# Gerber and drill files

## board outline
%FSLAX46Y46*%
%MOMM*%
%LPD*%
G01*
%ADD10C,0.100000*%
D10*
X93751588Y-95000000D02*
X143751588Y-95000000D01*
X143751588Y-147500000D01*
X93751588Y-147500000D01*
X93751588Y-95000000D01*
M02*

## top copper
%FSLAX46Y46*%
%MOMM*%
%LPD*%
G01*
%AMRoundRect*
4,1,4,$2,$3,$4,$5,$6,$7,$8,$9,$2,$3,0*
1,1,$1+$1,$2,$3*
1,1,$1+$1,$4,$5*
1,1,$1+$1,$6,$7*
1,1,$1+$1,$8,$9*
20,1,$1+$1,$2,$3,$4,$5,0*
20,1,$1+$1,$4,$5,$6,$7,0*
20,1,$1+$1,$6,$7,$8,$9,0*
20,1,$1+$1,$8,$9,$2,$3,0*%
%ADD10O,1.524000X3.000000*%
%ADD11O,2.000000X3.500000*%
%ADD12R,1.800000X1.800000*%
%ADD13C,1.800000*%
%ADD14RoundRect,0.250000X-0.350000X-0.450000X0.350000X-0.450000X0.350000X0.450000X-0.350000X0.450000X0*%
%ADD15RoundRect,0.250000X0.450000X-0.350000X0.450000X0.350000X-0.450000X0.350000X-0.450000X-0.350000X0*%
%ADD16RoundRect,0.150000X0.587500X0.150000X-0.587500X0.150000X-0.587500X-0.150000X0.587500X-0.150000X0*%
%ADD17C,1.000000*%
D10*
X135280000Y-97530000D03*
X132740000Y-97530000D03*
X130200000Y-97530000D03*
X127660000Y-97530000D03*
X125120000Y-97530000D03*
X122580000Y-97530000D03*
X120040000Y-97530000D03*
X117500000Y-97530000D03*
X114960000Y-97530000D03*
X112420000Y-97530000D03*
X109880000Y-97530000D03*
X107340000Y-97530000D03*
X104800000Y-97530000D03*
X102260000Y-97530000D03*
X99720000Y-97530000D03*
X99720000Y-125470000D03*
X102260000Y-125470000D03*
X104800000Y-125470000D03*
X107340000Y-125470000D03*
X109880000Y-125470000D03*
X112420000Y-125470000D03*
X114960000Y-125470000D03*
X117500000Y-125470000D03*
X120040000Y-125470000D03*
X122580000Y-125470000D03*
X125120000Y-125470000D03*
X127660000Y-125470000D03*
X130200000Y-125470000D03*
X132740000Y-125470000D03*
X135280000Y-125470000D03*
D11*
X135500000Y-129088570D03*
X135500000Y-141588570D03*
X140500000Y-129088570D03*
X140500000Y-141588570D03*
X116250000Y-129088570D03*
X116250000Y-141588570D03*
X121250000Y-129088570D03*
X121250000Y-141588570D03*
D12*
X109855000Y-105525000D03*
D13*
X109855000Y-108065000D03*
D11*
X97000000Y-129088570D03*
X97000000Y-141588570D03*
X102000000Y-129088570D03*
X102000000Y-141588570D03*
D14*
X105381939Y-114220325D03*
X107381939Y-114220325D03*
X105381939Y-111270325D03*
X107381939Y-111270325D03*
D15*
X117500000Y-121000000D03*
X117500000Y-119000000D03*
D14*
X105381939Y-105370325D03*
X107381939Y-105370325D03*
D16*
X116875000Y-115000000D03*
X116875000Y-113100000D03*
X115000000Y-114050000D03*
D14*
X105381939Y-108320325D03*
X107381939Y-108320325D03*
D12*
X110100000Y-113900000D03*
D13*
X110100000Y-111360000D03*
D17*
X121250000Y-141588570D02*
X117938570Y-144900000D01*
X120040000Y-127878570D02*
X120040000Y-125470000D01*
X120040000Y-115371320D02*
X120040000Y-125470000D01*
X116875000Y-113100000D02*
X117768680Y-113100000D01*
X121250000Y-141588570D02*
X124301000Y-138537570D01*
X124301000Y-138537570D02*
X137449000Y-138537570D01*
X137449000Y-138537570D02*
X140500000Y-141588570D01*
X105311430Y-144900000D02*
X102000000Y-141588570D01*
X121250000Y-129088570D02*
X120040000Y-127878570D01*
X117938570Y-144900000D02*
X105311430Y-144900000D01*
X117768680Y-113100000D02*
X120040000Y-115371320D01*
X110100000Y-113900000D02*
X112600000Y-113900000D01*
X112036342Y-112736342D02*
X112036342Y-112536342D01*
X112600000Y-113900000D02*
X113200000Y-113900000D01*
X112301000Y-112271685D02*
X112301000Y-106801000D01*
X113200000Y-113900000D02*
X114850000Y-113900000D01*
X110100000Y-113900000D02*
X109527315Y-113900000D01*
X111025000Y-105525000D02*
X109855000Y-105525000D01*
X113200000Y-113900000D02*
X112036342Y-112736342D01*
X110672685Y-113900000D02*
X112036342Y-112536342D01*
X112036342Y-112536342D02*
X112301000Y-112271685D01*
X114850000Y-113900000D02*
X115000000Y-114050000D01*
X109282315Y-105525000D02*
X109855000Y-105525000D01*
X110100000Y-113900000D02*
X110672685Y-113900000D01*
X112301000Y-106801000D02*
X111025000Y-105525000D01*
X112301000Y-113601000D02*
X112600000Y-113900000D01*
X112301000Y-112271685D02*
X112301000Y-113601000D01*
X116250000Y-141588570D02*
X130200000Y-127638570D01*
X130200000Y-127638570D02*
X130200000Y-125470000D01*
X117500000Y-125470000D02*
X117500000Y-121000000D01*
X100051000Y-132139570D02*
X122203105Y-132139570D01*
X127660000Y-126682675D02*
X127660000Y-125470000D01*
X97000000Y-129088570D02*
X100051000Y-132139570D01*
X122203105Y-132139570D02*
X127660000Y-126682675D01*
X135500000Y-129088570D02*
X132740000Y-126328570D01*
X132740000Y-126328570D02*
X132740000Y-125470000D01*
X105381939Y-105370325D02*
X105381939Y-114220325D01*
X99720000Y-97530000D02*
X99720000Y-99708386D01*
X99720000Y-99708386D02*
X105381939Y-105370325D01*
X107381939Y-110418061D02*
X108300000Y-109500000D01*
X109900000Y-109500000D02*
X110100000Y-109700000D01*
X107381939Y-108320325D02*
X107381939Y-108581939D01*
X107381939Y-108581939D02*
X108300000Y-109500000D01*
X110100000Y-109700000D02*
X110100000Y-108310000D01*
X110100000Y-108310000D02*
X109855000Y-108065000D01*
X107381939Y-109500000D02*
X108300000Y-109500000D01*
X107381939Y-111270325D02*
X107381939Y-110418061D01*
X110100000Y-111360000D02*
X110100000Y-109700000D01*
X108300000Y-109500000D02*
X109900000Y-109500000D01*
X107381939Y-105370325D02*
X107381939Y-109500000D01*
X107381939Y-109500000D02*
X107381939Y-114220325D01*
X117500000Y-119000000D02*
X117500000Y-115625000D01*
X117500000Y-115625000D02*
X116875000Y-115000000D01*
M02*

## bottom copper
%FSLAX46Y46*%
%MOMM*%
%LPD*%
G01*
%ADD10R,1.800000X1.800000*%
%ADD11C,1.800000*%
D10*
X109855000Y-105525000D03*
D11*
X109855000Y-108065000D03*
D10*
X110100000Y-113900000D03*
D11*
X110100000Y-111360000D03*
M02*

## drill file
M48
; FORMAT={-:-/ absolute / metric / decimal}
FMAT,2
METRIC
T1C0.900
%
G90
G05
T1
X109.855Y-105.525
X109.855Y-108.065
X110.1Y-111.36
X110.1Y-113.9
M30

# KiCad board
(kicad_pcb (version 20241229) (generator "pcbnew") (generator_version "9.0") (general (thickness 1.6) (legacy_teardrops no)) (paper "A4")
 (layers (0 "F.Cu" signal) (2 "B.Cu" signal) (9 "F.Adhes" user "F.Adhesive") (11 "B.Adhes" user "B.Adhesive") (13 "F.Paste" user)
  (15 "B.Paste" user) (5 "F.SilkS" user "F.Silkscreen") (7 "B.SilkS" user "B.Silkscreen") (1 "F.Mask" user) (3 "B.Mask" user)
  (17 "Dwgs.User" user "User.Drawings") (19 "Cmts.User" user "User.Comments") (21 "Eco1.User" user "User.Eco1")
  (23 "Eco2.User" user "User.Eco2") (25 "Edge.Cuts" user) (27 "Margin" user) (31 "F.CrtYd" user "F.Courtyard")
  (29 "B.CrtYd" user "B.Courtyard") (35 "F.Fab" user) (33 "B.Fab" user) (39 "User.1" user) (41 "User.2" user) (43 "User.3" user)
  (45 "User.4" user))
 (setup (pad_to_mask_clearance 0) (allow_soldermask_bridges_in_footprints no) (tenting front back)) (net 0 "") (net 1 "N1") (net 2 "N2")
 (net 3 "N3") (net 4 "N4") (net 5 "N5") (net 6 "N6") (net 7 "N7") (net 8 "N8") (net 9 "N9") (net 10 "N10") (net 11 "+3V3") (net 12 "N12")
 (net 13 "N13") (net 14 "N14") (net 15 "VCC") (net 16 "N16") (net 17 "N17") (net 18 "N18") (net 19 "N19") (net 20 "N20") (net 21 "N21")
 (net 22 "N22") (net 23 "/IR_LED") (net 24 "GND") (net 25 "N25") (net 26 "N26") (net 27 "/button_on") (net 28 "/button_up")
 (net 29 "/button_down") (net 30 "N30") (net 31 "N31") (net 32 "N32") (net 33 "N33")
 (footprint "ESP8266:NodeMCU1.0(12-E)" (layer "F.Cu") (at 117.5 111.5 -90)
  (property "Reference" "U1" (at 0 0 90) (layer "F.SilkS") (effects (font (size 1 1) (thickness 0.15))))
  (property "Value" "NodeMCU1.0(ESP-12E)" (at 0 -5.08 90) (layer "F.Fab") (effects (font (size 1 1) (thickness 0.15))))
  (pad "1" smd oval (at -13.97 -17.78 270) (size 3 1.524) (layers "F.Cu" "F.Mask" "F.Paste") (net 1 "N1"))
  (pad "2" smd oval (at -13.97 -15.24 270) (size 3 1.524) (layers "F.Cu" "F.Mask" "F.Paste") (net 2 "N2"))
  (pad "3" smd oval (at -13.97 -12.7 270) (size 3 1.524) (layers "F.Cu" "F.Mask" "F.Paste") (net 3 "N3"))
  (pad "4" smd oval (at -13.97 -10.16 270) (size 3 1.524) (layers "F.Cu" "F.Mask" "F.Paste") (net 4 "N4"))
  (pad "5" smd oval (at -13.97 -7.62 270) (size 3 1.524) (layers "F.Cu" "F.Mask" "F.Paste") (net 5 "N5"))
  (pad "6" smd oval (at -13.97 -5.08 270) (size 3 1.524) (layers "F.Cu" "F.Mask" "F.Paste") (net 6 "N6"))
  (pad "7" smd oval (at -13.97 -2.54 270) (size 3 1.524) (layers "F.Cu" "F.Mask" "F.Paste") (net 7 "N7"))
  (pad "8" smd oval (at -13.97 0 270) (size 3 1.524) (layers "F.Cu" "F.Mask" "F.Paste") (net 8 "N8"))
  (pad "9" smd oval (at -13.97 2.54 270) (size 3 1.524) (layers "F.Cu" "F.Mask" "F.Paste") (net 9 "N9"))
  (pad "10" smd oval (at -13.97 5.08 270) (size 3 1.524) (layers "F.Cu" "F.Mask" "F.Paste") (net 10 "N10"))
  (pad "11" smd oval (at -13.97 7.62 270) (size 3 1.524) (layers "F.Cu" "F.Mask" "F.Paste") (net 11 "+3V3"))
  (pad "12" smd oval (at -13.97 10.16 270) (size 3 1.524) (layers "F.Cu" "F.Mask" "F.Paste") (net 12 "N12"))
  (pad "13" smd oval (at -13.97 12.7 270) (size 3 1.524) (layers "F.Cu" "F.Mask" "F.Paste") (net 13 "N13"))
  (pad "14" smd oval (at -13.97 15.24 270) (size 3 1.524) (layers "F.Cu" "F.Mask" "F.Paste") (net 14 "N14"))
  (pad "15" smd oval (at -13.97 17.78 270) (size 3 1.524) (layers "F.Cu" "F.Mask" "F.Paste") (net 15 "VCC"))
  (pad "16" smd oval (at 13.97 17.78 270) (size 3 1.524) (layers "F.Cu" "F.Mask" "F.Paste") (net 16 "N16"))
  (pad "17" smd oval (at 13.97 15.24 270) (size 3 1.524) (layers "F.Cu" "F.Mask" "F.Paste") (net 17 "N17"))
  (pad "18" smd oval (at 13.97 12.7 270) (size 3 1.524) (layers "F.Cu" "F.Mask" "F.Paste") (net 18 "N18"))
  (pad "19" smd oval (at 13.97 10.16 270) (size 3 1.524) (layers "F.Cu" "F.Mask" "F.Paste") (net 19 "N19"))
  (pad "20" smd oval (at 13.97 7.62 270) (size 3 1.524) (layers "F.Cu" "F.Mask" "F.Paste") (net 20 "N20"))
  (pad "21" smd oval (at 13.97 5.08 270) (size 3 1.524) (layers "F.Cu" "F.Mask" "F.Paste") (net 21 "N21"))
  (pad "22" smd oval (at 13.97 2.54 270) (size 3 1.524) (layers "F.Cu" "F.Mask" "F.Paste") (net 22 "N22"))
  (pad "23" smd oval (at 13.97 0 270) (size 3 1.524) (layers "F.Cu" "F.Mask" "F.Paste") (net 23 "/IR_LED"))
  (pad "24" smd oval (at 13.97 -2.54 270) (size 3 1.524) (layers "F.Cu" "F.Mask" "F.Paste") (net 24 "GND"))
  (pad "25" smd oval (at 13.97 -5.08 270) (size 3 1.524) (layers "F.Cu" "F.Mask" "F.Paste") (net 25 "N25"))
  (pad "26" smd oval (at 13.97 -7.62 270) (size 3 1.524) (layers "F.Cu" "F.Mask" "F.Paste") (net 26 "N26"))
  (pad "27" smd oval (at 13.97 -10.16 270) (size 3 1.524) (layers "F.Cu" "F.Mask" "F.Paste") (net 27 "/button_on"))
  (pad "28" smd oval (at 13.97 -12.7 270) (size 3 1.524) (layers "F.Cu" "F.Mask" "F.Paste") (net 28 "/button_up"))
  (pad "29" smd oval (at 13.97 -15.24 270) (size 3 1.524) (layers "F.Cu" "F.Mask" "F.Paste") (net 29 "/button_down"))
  (pad "30" smd oval (at 13.97 -17.78 270) (size 3 1.524) (layers "F.Cu" "F.Mask" "F.Paste") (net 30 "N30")))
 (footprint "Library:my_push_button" (layer "F.Cu") (at 138 135.33857)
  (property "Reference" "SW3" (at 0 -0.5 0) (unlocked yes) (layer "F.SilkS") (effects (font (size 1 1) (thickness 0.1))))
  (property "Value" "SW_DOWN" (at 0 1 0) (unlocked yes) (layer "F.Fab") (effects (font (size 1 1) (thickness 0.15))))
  (pad "1" smd oval (at -2.5 -6.25) (size 2 3.5) (layers "F.Cu" "F.Mask" "F.Paste") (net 29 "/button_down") (thermal_bridge_angle 45))
  (pad "1" smd oval (at -2.5 6.25) (size 2 3.5) (layers "F.Cu" "F.Mask" "F.Paste") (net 29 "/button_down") (thermal_bridge_angle 45))
  (pad "2" smd oval (at 2.5 -6.25) (size 2 3.5) (layers "F.Cu" "F.Mask" "F.Paste") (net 24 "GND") (thermal_bridge_angle 45))
  (pad "2" smd oval (at 2.5 6.25) (size 2 3.5) (layers "F.Cu" "F.Mask" "F.Paste") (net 24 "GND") (thermal_bridge_angle 45)))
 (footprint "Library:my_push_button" (layer "F.Cu") (at 118.75 135.33857)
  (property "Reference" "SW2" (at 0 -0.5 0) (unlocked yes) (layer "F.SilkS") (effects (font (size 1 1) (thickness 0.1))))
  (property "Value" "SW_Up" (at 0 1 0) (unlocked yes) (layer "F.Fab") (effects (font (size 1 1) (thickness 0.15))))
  (pad "1" smd oval (at -2.5 -6.25) (size 2 3.5) (layers "F.Cu" "F.Mask" "F.Paste") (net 28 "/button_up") (thermal_bridge_angle 45))
  (pad "1" smd oval (at -2.5 6.25) (size 2 3.5) (layers "F.Cu" "F.Mask" "F.Paste") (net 28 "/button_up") (thermal_bridge_angle 45))
  (pad "2" smd oval (at 2.5 -6.25) (size 2 3.5) (layers "F.Cu" "F.Mask" "F.Paste") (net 24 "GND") (thermal_bridge_angle 45))
  (pad "2" smd oval (at 2.5 6.25) (size 2 3.5) (layers "F.Cu" "F.Mask" "F.Paste") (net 24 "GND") (thermal_bridge_angle 45)))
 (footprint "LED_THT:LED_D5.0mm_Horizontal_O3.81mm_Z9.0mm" (layer "F.Cu") (at 109.855 105.525 -90)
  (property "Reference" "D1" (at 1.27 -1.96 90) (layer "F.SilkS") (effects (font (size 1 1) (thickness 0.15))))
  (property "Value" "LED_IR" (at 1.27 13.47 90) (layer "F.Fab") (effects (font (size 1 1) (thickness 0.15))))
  (pad "1" thru_hole rect (at 0 0 270) (size 1.8 1.8) (drill 0.9) (layers "*.Cu" "*.Mask") (remove_unused_layers no) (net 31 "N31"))
  (pad "2" thru_hole circle (at 2.54 0 270) (size 1.8 1.8) (drill 0.9) (layers "*.Cu" "*.Mask") (remove_unused_layers no) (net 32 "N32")))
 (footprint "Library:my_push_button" (layer "F.Cu") (at 99.5 135.33857)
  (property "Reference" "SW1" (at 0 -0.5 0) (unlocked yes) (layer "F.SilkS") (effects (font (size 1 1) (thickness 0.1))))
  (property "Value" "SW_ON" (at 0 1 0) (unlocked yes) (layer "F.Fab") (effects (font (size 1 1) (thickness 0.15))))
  (pad "1" smd oval (at -2.5 -6.25) (size 2 3.5) (layers "F.Cu" "F.Mask" "F.Paste") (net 27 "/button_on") (thermal_bridge_angle 45))
  (pad "1" smd oval (at -2.5 6.25) (size 2 3.5) (layers "F.Cu" "F.Mask" "F.Paste") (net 27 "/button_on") (thermal_bridge_angle 45))
  (pad "2" smd oval (at 2.5 -6.25) (size 2 3.5) (layers "F.Cu" "F.Mask" "F.Paste") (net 24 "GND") (thermal_bridge_angle 45))
  (pad "2" smd oval (at 2.5 6.25) (size 2 3.5) (layers "F.Cu" "F.Mask" "F.Paste") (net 24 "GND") (thermal_bridge_angle 45))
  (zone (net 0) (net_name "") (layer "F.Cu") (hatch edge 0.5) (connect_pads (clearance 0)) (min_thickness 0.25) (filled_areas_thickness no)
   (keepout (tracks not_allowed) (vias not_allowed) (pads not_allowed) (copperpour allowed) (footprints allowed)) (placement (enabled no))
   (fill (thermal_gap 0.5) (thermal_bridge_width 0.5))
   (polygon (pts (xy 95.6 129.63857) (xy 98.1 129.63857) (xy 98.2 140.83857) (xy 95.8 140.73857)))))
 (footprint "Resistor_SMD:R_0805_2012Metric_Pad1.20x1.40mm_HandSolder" (layer "F.Cu") (at 106.381939 114.220325)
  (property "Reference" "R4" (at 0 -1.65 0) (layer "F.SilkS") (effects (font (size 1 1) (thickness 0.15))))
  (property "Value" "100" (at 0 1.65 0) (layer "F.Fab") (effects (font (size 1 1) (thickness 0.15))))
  (pad "1" smd roundrect (at -1 0) (size 1.2 1.4) (layers "F.Cu" "F.Mask" "F.Paste") (roundrect_rratio 0.208333) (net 15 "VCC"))
  (pad "2" smd roundrect (at 1 0) (size 1.2 1.4) (layers "F.Cu" "F.Mask" "F.Paste") (roundrect_rratio 0.208333) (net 32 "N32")))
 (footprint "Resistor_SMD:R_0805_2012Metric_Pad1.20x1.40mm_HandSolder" (layer "F.Cu") (at 106.381939 111.270325)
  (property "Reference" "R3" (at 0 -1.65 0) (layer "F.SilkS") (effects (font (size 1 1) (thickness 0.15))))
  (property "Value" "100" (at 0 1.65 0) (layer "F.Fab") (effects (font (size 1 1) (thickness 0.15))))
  (pad "1" smd roundrect (at -1 0) (size 1.2 1.4) (layers "F.Cu" "F.Mask" "F.Paste") (roundrect_rratio 0.208333) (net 15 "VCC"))
  (pad "2" smd roundrect (at 1 0) (size 1.2 1.4) (layers "F.Cu" "F.Mask" "F.Paste") (roundrect_rratio 0.208333) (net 32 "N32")))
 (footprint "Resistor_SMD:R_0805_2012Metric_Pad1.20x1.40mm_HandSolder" (layer "F.Cu") (at 117.5 120 90)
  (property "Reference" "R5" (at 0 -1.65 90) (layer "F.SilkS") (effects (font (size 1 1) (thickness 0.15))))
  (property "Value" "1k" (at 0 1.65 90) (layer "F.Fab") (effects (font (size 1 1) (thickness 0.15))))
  (pad "1" smd roundrect (at -1 0 90) (size 1.2 1.4) (layers "F.Cu" "F.Mask" "F.Paste") (roundrect_rratio 0.208333) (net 23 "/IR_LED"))
  (pad "2" smd roundrect (at 1 0 90) (size 1.2 1.4) (layers "F.Cu" "F.Mask" "F.Paste") (roundrect_rratio 0.208333) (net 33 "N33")))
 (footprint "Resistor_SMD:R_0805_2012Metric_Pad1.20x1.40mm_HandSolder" (layer "F.Cu") (at 106.381939 105.370325)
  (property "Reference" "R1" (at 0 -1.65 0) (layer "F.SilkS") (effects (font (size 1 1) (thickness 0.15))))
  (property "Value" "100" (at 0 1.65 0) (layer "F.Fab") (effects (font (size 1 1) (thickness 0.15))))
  (pad "1" smd roundrect (at -1 0) (size 1.2 1.4) (layers "F.Cu" "F.Mask" "F.Paste") (roundrect_rratio 0.208333) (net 15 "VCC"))
  (pad "2" smd roundrect (at 1 0) (size 1.2 1.4) (layers "F.Cu" "F.Mask" "F.Paste") (roundrect_rratio 0.208333) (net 32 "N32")))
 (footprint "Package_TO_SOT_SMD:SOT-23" (layer "F.Cu") (at 115.9375 114.05 180)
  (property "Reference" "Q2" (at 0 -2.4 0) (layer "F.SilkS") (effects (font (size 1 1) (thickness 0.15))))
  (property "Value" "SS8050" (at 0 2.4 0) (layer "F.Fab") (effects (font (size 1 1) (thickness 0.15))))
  (pad "1" smd roundrect (at -0.9375 -0.95 180) (size 1.475 0.6) (layers "F.Cu" "F.Mask" "F.Paste") (roundrect_rratio 0.25) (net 33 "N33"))
  (pad "2" smd roundrect (at -0.9375 0.95 180) (size 1.475 0.6) (layers "F.Cu" "F.Mask" "F.Paste") (roundrect_rratio 0.25) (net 24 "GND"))
  (pad "3" smd roundrect (at 0.9375 0 180) (size 1.475 0.6) (layers "F.Cu" "F.Mask" "F.Paste") (roundrect_rratio 0.25) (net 31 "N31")))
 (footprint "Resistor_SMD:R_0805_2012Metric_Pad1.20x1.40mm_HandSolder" (layer "F.Cu") (at 106.381939 108.320325)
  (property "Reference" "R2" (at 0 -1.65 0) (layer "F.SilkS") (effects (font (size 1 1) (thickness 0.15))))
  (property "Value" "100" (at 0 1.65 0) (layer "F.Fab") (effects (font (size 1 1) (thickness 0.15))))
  (pad "1" smd roundrect (at -1 0) (size 1.2 1.4) (layers "F.Cu" "F.Mask" "F.Paste") (roundrect_rratio 0.208333) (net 15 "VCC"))
  (pad "2" smd roundrect (at 1 0) (size 1.2 1.4) (layers "F.Cu" "F.Mask" "F.Paste") (roundrect_rratio 0.208333) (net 32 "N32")))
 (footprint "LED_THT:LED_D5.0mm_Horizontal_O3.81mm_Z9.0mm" (layer "B.Cu") (at 110.1 113.9 90)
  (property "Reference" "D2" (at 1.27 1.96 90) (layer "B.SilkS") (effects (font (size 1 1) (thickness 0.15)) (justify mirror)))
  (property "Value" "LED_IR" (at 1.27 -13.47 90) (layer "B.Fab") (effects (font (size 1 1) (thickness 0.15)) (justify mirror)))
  (pad "1" thru_hole rect (at 0 0 90) (size 1.8 1.8) (drill 0.9) (layers "*.Cu" "*.Mask") (remove_unused_layers no) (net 31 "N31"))
  (pad "2" thru_hole circle (at 2.54 0 90) (size 1.8 1.8) (drill 0.9) (layers "*.Cu" "*.Mask") (remove_unused_layers no) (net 32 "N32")))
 (gr_rect (start 93.751588 95) (end 143.751588 147.5) (stroke (width 0.1) (type solid)) (fill no) (layer "Edge.Cuts"))
 (segment (start 121.25 141.58857) (end 117.93857 144.9) (width 1) (layer "F.Cu") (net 24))
 (segment (start 120.04 127.87857) (end 120.04 125.47) (width 1) (layer "F.Cu") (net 24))
 (segment (start 120.04 115.37132) (end 120.04 125.47) (width 1) (layer "F.Cu") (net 24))
 (segment (start 116.875 113.1) (end 117.76868 113.1) (width 1) (layer "F.Cu") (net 24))
 (segment (start 121.25 141.58857) (end 124.301 138.53757) (width 1) (layer "F.Cu") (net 24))
 (segment (start 124.301 138.53757) (end 137.449 138.53757) (width 1) (layer "F.Cu") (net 24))
 (segment (start 137.449 138.53757) (end 140.5 141.58857) (width 1) (layer "F.Cu") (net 24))
 (segment (start 105.31143 144.9) (end 102 141.58857) (width 1) (layer "F.Cu") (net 24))
 (segment (start 121.25 129.08857) (end 120.04 127.87857) (width 1) (layer "F.Cu") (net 24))
 (segment (start 117.93857 144.9) (end 105.31143 144.9) (width 1) (locked yes) (layer "F.Cu") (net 24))
 (segment (start 117.76868 113.1) (end 120.04 115.37132) (width 1) (layer "F.Cu") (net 24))
 (segment (start 110.1 113.9) (end 112.6 113.9) (width 1) (layer "F.Cu") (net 31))
 (segment (start 112.036342 112.736342) (end 112.036342 112.536342) (width 1) (layer "F.Cu") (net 31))
 (segment (start 112.6 113.9) (end 113.2 113.9) (width 1) (layer "F.Cu") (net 31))
 (segment (start 112.301 112.271685) (end 112.301 106.801) (width 1) (layer "F.Cu") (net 31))
 (segment (start 113.2 113.9) (end 114.85 113.9) (width 1) (layer "F.Cu") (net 31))
 (segment (start 110.1 113.9) (end 109.527315 113.9) (width 1) (layer "F.Cu") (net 31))
 (segment (start 111.025 105.525) (end 109.855 105.525) (width 1) (layer "F.Cu") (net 31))
 (segment (start 113.2 113.9) (end 112.036342 112.736342) (width 1) (layer "F.Cu") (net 31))
 (segment (start 110.672685 113.9) (end 112.036342 112.536342) (width 1) (layer "F.Cu") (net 31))
 (segment (start 112.036342 112.536342) (end 112.301 112.271685) (width 1) (layer "F.Cu") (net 31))
 (segment (start 114.85 113.9) (end 115 114.05) (width 1) (layer "F.Cu") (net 31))
 (segment (start 109.282315 105.525) (end 109.855 105.525) (width 1) (layer "F.Cu") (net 31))
 (segment (start 110.1 113.9) (end 110.672685 113.9) (width 1) (layer "F.Cu") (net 31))
 (segment (start 112.301 106.801) (end 111.025 105.525) (width 1) (layer "F.Cu") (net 31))
 (segment (start 112.301 113.601) (end 112.6 113.9) (width 1) (layer "F.Cu") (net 31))
 (segment (start 112.301 112.271685) (end 112.301 113.601) (width 1) (layer "F.Cu") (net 31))
 (segment (start 116.25 141.58857) (end 130.2 127.63857) (width 1) (layer "F.Cu") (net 28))
 (segment (start 130.2 127.63857) (end 130.2 125.47) (width 1) (layer "F.Cu") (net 28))
 (segment (start 117.5 125.47) (end 117.5 121) (width 1) (layer "F.Cu") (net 23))
 (segment (start 100.051 132.13957) (end 122.203105 132.13957) (width 1) (layer "F.Cu") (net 27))
 (segment (start 127.66 126.682675) (end 127.66 125.47) (width 1) (layer "F.Cu") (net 27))
 (segment (start 97 129.08857) (end 100.051 132.13957) (width 1) (layer "F.Cu") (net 27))
 (segment (start 122.203105 132.13957) (end 127.66 126.682675) (width 1) (layer "F.Cu") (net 27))
 (segment (start 135.5 129.08857) (end 132.74 126.32857) (width 1) (layer "F.Cu") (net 29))
 (segment (start 132.74 126.32857) (end 132.74 125.47) (width 1) (layer "F.Cu") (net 29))
 (segment (start 105.381939 105.370325) (end 105.381939 114.220325) (width 1) (layer "F.Cu") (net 15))
 (segment (start 99.72 97.53) (end 99.72 99.708386) (width 1) (layer "F.Cu") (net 15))
 (segment (start 99.72 99.708386) (end 105.381939 105.370325) (width 1) (layer "F.Cu") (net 15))
 (segment (start 107.381939 110.418061) (end 108.3 109.5) (width 1) (layer "F.Cu") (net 32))
 (segment (start 109.9 109.5) (end 110.1 109.7) (width 1) (layer "F.Cu") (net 32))
 (segment (start 107.381939 108.320325) (end 107.381939 108.581939) (width 1) (layer "F.Cu") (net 32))
 (segment (start 107.381939 108.581939) (end 108.3 109.5) (width 1) (layer "F.Cu") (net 32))
 (segment (start 110.1 109.7) (end 110.1 108.31) (width 1) (layer "F.Cu") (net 32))
 (segment (start 110.1 108.31) (end 109.855 108.065) (width 1) (layer "F.Cu") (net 32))
 (segment (start 107.381939 109.5) (end 108.3 109.5) (width 1) (layer "F.Cu") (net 32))
 (segment (start 107.381939 111.270325) (end 107.381939 110.418061) (width 1) (layer "F.Cu") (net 32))
 (segment (start 110.1 111.36) (end 110.1 109.7) (width 1) (layer "F.Cu") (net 32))
 (segment (start 108.3 109.5) (end 109.9 109.5) (width 1) (layer "F.Cu") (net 32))
 (segment (start 107.381939 105.370325) (end 107.381939 109.5) (width 1) (layer "F.Cu") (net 32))
 (segment (start 107.381939 109.5) (end 107.381939 114.220325) (width 1) (layer "F.Cu") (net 32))
 (segment (start 117.5 119) (end 117.5 115.625) (width 1) (layer "F.Cu") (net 33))
 (segment (start 117.5 115.625) (end 116.875 115) (width 1) (layer "F.Cu") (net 33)))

